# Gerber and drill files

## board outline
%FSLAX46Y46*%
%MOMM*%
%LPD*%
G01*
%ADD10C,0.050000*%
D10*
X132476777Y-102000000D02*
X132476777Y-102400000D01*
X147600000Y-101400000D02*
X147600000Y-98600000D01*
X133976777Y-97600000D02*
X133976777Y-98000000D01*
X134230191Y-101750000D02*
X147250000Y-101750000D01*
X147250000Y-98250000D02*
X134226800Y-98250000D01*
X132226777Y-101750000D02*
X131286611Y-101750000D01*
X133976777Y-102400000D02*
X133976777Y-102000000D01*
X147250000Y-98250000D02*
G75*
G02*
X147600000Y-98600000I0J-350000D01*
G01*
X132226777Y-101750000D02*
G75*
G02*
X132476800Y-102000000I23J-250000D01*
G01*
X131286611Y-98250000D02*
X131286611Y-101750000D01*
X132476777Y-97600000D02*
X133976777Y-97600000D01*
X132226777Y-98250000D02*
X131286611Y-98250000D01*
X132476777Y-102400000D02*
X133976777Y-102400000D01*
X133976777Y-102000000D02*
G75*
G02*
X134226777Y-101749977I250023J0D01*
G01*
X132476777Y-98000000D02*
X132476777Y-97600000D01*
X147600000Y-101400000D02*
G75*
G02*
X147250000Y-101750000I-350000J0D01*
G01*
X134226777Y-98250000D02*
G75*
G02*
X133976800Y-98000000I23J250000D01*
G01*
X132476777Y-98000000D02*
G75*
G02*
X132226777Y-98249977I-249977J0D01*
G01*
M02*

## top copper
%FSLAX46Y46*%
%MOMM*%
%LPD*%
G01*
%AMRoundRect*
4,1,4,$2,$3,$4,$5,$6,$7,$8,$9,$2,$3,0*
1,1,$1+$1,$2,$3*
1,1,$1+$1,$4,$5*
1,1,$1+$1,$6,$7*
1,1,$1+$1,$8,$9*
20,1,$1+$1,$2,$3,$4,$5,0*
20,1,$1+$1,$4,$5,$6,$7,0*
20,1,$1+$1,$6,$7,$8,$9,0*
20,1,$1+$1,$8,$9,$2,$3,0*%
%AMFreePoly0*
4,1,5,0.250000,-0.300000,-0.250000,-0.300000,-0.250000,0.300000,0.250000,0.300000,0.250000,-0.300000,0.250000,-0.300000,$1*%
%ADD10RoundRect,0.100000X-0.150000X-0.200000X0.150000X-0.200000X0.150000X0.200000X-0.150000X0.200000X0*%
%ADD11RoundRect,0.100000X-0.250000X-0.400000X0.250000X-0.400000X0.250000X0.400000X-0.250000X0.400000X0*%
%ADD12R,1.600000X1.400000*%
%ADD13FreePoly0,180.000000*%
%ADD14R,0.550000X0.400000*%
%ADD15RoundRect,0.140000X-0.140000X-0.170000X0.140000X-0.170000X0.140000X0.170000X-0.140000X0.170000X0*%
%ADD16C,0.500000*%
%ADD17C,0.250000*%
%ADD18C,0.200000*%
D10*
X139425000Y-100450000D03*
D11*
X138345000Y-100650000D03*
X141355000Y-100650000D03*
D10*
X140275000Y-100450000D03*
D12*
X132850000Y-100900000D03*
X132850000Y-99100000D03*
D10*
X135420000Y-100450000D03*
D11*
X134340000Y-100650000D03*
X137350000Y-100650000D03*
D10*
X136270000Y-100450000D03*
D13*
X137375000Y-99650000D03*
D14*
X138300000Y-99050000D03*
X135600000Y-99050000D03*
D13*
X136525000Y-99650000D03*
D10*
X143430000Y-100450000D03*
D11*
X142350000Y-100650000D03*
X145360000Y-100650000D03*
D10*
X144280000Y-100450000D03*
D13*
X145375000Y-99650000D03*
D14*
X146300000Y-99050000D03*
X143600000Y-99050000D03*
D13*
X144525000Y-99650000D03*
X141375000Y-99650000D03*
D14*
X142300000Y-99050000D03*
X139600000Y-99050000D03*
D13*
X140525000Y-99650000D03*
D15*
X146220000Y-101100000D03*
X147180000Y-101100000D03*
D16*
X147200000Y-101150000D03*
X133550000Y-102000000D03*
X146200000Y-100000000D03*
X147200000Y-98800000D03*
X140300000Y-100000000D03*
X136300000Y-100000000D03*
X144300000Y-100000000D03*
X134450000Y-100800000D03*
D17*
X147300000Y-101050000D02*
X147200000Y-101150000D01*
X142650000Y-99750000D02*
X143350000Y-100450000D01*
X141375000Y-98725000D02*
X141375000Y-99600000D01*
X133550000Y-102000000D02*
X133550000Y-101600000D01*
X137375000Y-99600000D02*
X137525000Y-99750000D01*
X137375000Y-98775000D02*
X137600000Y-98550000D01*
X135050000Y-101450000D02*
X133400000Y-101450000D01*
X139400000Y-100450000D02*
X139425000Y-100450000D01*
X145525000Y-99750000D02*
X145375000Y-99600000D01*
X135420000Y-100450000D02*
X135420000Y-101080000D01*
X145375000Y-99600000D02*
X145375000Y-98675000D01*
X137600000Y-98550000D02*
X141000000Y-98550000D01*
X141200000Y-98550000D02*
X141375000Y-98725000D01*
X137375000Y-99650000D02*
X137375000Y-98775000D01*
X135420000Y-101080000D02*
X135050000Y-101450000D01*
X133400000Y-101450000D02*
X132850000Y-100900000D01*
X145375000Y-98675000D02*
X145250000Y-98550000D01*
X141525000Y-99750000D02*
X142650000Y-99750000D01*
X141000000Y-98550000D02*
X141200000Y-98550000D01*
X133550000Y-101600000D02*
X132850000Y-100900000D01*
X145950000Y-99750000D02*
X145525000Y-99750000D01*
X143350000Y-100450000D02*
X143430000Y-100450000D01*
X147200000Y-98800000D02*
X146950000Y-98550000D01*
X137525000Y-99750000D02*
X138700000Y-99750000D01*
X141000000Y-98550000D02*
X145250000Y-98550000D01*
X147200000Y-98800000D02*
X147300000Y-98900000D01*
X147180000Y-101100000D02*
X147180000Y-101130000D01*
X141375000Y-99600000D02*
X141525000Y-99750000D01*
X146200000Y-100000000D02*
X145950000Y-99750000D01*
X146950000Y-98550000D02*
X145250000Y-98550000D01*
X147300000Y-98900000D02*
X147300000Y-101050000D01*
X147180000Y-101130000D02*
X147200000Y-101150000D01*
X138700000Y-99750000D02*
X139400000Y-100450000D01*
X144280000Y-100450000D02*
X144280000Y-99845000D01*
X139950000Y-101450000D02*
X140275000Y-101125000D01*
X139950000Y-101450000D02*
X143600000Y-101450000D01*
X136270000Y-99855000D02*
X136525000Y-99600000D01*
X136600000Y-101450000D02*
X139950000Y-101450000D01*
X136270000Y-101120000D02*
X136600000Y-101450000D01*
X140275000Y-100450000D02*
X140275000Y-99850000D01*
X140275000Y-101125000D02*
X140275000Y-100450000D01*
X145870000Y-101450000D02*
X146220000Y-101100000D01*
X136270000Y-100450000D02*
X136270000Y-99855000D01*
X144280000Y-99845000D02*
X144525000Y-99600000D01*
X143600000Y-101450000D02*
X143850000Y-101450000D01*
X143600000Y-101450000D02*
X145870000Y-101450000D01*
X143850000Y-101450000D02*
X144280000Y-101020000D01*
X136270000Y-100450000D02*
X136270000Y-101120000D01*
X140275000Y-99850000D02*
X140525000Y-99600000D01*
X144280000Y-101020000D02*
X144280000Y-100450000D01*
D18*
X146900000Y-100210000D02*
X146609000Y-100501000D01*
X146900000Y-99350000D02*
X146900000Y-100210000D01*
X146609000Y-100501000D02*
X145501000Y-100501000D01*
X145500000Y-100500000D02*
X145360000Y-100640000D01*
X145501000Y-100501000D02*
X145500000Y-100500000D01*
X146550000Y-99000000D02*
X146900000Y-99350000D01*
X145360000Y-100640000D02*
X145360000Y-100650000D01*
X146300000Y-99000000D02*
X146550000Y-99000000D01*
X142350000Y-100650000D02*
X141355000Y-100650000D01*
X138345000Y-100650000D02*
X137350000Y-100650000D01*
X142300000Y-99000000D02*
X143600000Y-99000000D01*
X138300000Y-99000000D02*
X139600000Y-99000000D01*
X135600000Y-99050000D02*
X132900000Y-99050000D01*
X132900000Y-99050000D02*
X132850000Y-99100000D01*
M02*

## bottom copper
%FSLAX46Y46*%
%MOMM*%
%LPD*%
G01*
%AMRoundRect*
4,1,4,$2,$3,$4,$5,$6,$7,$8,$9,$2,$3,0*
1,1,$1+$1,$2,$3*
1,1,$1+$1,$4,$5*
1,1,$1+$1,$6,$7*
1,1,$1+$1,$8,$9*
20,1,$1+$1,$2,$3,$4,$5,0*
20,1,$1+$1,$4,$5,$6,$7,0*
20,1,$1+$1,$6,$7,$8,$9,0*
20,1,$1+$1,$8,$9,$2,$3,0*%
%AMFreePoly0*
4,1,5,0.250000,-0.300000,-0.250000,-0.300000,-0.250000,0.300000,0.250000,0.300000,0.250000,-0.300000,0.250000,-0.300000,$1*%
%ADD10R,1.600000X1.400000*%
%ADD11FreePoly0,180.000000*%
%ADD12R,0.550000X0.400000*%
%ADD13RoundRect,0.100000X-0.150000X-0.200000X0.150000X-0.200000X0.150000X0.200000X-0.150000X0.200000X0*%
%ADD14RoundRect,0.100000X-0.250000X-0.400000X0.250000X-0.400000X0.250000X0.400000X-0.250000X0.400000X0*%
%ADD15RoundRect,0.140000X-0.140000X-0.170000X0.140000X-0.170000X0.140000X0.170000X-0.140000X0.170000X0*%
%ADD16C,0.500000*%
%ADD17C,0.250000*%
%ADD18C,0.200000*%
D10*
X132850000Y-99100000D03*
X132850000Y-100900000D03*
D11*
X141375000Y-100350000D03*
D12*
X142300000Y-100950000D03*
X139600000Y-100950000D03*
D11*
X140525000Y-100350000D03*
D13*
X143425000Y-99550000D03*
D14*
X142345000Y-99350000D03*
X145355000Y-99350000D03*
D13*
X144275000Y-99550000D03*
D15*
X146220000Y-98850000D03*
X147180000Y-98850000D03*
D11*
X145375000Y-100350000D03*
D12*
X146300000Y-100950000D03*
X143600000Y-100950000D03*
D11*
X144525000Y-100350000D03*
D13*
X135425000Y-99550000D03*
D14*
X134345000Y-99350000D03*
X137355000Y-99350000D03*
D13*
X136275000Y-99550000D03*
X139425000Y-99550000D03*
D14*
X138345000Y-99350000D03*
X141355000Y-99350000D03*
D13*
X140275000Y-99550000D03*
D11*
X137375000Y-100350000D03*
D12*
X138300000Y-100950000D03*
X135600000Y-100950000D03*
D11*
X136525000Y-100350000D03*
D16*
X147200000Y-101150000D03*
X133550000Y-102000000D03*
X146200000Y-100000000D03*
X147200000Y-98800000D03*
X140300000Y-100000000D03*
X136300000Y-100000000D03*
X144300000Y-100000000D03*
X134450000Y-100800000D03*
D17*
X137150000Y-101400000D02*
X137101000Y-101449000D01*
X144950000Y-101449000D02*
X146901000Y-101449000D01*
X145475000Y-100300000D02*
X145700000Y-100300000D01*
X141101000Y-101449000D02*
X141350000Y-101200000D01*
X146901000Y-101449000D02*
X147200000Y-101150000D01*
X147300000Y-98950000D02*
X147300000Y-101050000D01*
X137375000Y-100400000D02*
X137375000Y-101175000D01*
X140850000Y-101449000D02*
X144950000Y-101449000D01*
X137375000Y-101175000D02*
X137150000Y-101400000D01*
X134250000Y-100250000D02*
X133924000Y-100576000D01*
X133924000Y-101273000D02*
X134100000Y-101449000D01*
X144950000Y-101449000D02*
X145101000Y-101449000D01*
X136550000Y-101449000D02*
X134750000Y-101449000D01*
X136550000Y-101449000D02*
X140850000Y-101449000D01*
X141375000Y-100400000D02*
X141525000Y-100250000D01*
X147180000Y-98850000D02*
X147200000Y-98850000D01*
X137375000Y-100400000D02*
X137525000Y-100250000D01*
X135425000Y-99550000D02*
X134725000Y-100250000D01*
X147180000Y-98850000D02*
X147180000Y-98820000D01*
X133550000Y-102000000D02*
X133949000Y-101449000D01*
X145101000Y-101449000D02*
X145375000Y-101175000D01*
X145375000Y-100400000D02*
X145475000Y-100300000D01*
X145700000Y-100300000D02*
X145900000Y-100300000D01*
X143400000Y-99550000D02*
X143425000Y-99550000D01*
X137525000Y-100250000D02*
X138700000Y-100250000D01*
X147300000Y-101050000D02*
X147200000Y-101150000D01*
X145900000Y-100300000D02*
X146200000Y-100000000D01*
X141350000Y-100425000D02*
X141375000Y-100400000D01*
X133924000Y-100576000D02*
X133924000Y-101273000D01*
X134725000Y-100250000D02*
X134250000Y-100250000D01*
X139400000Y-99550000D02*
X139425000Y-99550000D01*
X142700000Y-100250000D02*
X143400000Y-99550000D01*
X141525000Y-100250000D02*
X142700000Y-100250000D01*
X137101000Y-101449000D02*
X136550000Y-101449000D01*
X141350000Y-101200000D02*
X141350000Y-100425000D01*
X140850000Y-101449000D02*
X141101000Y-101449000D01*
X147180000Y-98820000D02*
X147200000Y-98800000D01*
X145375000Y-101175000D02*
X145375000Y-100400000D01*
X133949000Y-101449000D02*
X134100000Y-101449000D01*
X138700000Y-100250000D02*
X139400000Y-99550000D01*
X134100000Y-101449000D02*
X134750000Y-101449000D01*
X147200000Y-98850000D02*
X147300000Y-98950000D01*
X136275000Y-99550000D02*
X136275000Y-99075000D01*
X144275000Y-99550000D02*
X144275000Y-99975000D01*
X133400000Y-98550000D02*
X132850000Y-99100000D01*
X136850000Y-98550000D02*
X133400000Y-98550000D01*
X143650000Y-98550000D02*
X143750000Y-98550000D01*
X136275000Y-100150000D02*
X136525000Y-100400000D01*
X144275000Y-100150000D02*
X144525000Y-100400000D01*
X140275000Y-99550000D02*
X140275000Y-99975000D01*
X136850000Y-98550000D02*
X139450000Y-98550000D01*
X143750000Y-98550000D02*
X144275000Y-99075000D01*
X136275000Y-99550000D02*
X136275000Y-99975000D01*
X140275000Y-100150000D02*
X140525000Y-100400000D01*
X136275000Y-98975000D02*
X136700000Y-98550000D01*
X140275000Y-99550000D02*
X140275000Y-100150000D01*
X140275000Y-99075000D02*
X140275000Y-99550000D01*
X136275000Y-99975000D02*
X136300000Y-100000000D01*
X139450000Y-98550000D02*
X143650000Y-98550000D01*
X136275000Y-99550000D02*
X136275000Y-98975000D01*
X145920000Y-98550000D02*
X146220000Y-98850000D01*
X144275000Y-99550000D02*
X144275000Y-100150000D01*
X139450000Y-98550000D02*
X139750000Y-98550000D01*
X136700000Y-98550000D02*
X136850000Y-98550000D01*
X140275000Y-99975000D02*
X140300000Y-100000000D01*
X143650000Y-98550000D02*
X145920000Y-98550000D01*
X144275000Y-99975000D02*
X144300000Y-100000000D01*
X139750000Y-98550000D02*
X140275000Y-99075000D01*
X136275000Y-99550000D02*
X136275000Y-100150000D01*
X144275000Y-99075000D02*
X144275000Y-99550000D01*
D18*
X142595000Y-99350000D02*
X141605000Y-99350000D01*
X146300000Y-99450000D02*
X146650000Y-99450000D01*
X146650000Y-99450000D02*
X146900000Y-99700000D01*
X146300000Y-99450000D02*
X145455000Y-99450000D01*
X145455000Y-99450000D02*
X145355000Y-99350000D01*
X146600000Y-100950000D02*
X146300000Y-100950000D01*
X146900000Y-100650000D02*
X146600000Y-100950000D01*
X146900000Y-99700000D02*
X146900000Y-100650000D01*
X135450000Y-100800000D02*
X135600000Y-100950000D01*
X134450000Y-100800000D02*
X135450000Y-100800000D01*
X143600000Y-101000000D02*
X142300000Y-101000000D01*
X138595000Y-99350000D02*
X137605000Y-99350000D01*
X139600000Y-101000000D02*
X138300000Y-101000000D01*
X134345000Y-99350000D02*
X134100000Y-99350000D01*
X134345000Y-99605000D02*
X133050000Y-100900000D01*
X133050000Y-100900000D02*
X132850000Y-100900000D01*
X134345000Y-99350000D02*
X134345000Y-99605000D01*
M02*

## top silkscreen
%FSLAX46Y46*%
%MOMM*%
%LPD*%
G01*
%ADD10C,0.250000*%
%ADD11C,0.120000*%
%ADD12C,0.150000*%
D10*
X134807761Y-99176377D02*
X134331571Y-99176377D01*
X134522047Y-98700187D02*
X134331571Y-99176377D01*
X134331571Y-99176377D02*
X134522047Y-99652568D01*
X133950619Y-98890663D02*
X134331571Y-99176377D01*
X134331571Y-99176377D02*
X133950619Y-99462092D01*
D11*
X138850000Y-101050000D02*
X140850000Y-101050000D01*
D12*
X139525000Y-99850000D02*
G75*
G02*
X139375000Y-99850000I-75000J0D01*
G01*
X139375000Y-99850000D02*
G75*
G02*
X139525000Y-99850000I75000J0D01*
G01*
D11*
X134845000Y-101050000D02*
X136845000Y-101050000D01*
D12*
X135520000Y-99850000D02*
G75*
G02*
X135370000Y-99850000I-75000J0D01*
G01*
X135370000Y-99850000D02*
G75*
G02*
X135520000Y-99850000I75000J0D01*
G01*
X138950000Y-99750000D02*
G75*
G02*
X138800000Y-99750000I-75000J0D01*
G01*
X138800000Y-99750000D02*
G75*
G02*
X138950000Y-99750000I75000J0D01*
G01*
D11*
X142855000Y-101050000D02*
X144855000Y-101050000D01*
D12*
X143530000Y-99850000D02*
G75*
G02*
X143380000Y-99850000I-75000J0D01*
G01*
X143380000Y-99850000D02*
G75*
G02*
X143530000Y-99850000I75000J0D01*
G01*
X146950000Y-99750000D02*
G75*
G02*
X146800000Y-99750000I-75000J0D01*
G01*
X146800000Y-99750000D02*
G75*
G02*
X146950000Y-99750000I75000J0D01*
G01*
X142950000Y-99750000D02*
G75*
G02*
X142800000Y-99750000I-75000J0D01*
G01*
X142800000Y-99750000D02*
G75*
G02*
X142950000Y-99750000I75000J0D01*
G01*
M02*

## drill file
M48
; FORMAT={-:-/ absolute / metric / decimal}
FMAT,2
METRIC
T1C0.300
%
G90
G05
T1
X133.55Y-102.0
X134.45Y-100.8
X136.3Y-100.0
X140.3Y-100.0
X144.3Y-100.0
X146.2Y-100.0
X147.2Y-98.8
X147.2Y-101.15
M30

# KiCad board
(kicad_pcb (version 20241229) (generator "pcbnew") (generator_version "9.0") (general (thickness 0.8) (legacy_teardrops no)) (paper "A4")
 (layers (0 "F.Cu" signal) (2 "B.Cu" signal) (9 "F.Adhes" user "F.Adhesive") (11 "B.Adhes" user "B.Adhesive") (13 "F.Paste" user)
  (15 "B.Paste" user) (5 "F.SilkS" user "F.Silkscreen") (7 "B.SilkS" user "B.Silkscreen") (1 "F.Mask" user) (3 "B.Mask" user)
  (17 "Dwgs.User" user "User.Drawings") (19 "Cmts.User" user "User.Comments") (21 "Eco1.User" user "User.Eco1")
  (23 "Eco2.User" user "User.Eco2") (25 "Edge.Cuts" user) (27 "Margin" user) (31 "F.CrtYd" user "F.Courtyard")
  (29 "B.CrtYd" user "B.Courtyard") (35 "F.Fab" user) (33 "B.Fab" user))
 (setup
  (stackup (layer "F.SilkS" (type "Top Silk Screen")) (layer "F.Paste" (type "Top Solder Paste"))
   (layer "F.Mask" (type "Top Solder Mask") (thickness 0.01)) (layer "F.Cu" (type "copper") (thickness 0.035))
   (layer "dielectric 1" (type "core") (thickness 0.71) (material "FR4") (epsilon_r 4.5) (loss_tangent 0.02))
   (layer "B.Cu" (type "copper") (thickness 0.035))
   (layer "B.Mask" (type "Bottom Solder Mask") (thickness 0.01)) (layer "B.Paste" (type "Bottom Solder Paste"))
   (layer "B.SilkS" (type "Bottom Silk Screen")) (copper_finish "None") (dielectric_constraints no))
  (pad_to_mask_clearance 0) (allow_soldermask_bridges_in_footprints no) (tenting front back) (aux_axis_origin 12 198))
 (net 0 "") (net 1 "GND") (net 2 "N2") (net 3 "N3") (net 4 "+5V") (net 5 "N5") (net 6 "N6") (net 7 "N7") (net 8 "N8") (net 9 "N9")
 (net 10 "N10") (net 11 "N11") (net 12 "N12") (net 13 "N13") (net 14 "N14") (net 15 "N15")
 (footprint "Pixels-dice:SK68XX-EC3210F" (layer "F.Cu") (at 139.85 100.65)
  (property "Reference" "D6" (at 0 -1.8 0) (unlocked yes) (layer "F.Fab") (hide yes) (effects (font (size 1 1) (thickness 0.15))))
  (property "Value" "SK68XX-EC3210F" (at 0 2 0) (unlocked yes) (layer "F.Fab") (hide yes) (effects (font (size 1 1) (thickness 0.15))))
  (fp_line (start -1 0.4) (end 1 0.4) (stroke (width 0.12) (type default)) (layer "F.SilkS"))
  (fp_circle (center -0.4 -0.8) (end -0.3 -0.8) (stroke (width 0.1) (type solid)) (fill yes) (layer "F.SilkS"))
  (pad "1" smd roundrect (at -0.425 -0.2) (size 0.5 0.6) (layers "F.Cu" "F.Mask" "F.Paste") (roundrect_rratio 0.2) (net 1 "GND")
   (thermal_bridge_angle 45))
  (pad "2" smd roundrect (at -1.505 0) (size 0.7 1) (layers "F.Cu" "F.Mask" "F.Paste") (roundrect_rratio 0.1428571429) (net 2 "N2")
   (thermal_bridge_angle 45))
  (pad "3" smd roundrect (at 1.505 0) (size 0.7 1) (layers "F.Cu" "F.Mask" "F.Paste") (roundrect_rratio 0.1428571429) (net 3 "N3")
   (thermal_bridge_angle 45))
  (pad "4" smd roundrect (at 0.425 -0.2) (size 0.5 0.6) (layers "F.Cu" "F.Mask" "F.Paste") (roundrect_rratio 0.2) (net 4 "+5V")
   (thermal_bridge_angle 45)))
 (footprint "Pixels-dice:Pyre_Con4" (layer "F.Cu") (at 132.85 100 90)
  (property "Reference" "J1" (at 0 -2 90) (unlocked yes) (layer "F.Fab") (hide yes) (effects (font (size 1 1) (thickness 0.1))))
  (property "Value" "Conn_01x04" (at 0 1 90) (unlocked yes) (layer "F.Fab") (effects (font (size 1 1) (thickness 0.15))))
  (pad "1" connect rect (at -0.9 0 90) (size 1.4 1.6) (layers "F.Cu" "F.Mask") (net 1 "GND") (thermal_bridge_angle 45))
  (pad "2" connect rect (at 0.9 0 90) (size 1.4 1.6) (layers "F.Cu" "F.Mask") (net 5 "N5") (thermal_bridge_angle 45))
  (pad "3" connect rect (at 0.9 0 90) (size 1.4 1.6) (layers "B.Cu" "B.Mask") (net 4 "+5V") (thermal_bridge_angle 45))
  (pad "4" connect rect (at -0.9 0 90) (size 1.4 1.6) (layers "B.Cu" "B.Mask") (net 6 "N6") (thermal_bridge_angle 45)))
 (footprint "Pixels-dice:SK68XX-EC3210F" (layer "F.Cu") (at 135.845 100.65)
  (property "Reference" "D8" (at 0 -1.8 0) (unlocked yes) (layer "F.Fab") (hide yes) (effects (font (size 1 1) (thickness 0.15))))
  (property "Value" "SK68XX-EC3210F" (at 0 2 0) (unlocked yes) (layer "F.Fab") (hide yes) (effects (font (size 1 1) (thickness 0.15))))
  (fp_line (start -1 0.4) (end 1 0.4) (stroke (width 0.12) (type default)) (layer "F.SilkS"))
  (fp_circle (center -0.4 -0.8) (end -0.3 -0.8) (stroke (width 0.1) (type solid)) (fill yes) (layer "F.SilkS"))
  (pad "1" smd roundrect (at -0.425 -0.2) (size 0.5 0.6) (layers "F.Cu" "F.Mask" "F.Paste") (roundrect_rratio 0.2) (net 1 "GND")
   (thermal_bridge_angle 45))
  (pad "2" smd roundrect (at -1.505 0) (size 0.7 1) (layers "F.Cu" "F.Mask" "F.Paste") (roundrect_rratio 0.1428571429) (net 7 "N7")
   (thermal_bridge_angle 45))
  (pad "3" smd roundrect (at 1.505 0) (size 0.7 1) (layers "F.Cu" "F.Mask" "F.Paste") (roundrect_rratio 0.1428571429) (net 2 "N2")
   (thermal_bridge_angle 45))
  (pad "4" smd roundrect (at 0.425 -0.2) (size 0.5 0.6) (layers "F.Cu" "F.Mask" "F.Paste") (roundrect_rratio 0.2) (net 4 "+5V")
   (thermal_bridge_angle 45)))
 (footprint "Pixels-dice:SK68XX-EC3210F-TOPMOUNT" (layer "F.Cu") (at 136.95 99.4 180)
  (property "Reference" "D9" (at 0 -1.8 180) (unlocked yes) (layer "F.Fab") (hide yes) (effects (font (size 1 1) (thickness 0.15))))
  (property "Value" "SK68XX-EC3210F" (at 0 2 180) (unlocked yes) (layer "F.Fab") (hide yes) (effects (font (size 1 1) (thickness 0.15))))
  (fp_circle (center -1.925 -0.35) (end -1.825 -0.35) (stroke (width 0.1) (type solid)) (fill yes) (layer "F.SilkS"))
  (pad "1" smd custom (at -0.425 -0.25 180) (size 0.5 0.6) (layers "F.Cu" "F.Mask" "F.Paste") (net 1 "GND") (thermal_bridge_angle 45)
   (options (clearance outline) (anchor rect)) (primitives))
  (pad "2" smd rect (at -1.35 0.35 180) (size 0.55 0.4) (layers "F.Cu" "F.Mask" "F.Paste") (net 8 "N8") (thermal_bridge_angle 45))
  (pad "3" smd rect (at 1.35 0.35 180) (size 0.55 0.4) (layers "F.Cu" "F.Mask" "F.Paste") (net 5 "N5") (thermal_bridge_angle 45))
  (pad "4" smd custom (at 0.425 -0.25 180) (size 0.5 0.6) (layers "F.Cu" "F.Mask" "F.Paste") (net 4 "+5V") (thermal_bridge_angle 45)
   (options (clearance outline) (anchor rect)) (primitives)))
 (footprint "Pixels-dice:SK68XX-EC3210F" (layer "F.Cu") (at 143.855 100.65)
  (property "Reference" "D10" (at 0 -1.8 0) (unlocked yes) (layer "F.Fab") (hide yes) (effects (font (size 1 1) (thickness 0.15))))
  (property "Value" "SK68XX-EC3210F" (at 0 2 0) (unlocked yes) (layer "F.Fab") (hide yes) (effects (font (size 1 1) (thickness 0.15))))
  (fp_line (start -1 0.4) (end 1 0.4) (stroke (width 0.12) (type default)) (layer "F.SilkS"))
  (fp_circle (center -0.4 -0.8) (end -0.3 -0.8) (stroke (width 0.1) (type solid)) (fill yes) (layer "F.SilkS"))
  (pad "1" smd roundrect (at -0.425 -0.2) (size 0.5 0.6) (layers "F.Cu" "F.Mask" "F.Paste") (roundrect_rratio 0.2) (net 1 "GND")
   (thermal_bridge_angle 45))
  (pad "2" smd roundrect (at -1.505 0) (size 0.7 1) (layers "F.Cu" "F.Mask" "F.Paste") (roundrect_rratio 0.1428571429) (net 3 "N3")
   (thermal_bridge_angle 45))
  (pad "3" smd roundrect (at 1.505 0) (size 0.7 1) (layers "F.Cu" "F.Mask" "F.Paste") (roundrect_rratio 0.1428571429) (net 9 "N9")
   (thermal_bridge_angle 45))
  (pad "4" smd roundrect (at 0.425 -0.2) (size 0.5 0.6) (layers "F.Cu" "F.Mask" "F.Paste") (roundrect_rratio 0.2) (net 4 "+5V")
   (thermal_bridge_angle 45)))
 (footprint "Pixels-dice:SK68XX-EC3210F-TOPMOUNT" (layer "F.Cu") (at 144.95 99.4 180)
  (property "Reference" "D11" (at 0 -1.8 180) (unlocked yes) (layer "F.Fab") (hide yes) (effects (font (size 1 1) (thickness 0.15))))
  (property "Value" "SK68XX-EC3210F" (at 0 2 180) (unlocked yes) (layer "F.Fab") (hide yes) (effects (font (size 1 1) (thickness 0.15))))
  (fp_circle (center -1.925 -0.35) (end -1.825 -0.35) (stroke (width 0.1) (type solid)) (fill yes) (layer "F.SilkS"))
  (pad "1" smd custom (at -0.425 -0.25 180) (size 0.5 0.6) (layers "F.Cu" "F.Mask" "F.Paste") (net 1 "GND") (thermal_bridge_angle 45)
   (options (clearance outline) (anchor rect)) (primitives))
  (pad "2" smd rect (at -1.35 0.35 180) (size 0.55 0.4) (layers "F.Cu" "F.Mask" "F.Paste") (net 9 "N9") (thermal_bridge_angle 45))
  (pad "3" smd rect (at 1.35 0.35 180) (size 0.55 0.4) (layers "F.Cu" "F.Mask" "F.Paste") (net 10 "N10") (thermal_bridge_angle 45))
  (pad "4" smd custom (at 0.425 -0.25 180) (size 0.5 0.6) (layers "F.Cu" "F.Mask" "F.Paste") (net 4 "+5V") (thermal_bridge_angle 45)
   (options (clearance outline) (anchor rect)) (primitives)))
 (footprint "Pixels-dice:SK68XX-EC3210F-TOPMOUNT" (layer "F.Cu") (at 140.95 99.4 180)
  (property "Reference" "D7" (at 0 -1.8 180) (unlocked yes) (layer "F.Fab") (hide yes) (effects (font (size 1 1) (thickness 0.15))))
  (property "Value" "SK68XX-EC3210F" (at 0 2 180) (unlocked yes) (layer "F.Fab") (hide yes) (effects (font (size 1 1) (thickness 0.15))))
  (fp_circle (center -1.925 -0.35) (end -1.825 -0.35) (stroke (width 0.1) (type solid)) (fill yes) (layer "F.SilkS"))
  (pad "1" smd custom (at -0.425 -0.25 180) (size 0.5 0.6) (layers "F.Cu" "F.Mask" "F.Paste") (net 1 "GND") (thermal_bridge_angle 45)
   (options (clearance outline) (anchor rect)) (primitives))
  (pad "2" smd rect (at -1.35 0.35 180) (size 0.55 0.4) (layers "F.Cu" "F.Mask" "F.Paste") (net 10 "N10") (thermal_bridge_angle 45))
  (pad "3" smd rect (at 1.35 0.35 180) (size 0.55 0.4) (layers "F.Cu" "F.Mask" "F.Paste") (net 8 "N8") (thermal_bridge_angle 45))
  (pad "4" smd custom (at 0.425 -0.25 180) (size 0.5 0.6) (layers "F.Cu" "F.Mask" "F.Paste") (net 4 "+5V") (thermal_bridge_angle 45)
   (options (clearance outline) (anchor rect)) (primitives)))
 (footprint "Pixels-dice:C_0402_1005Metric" (layer "F.Cu") (at 146.7 101.1)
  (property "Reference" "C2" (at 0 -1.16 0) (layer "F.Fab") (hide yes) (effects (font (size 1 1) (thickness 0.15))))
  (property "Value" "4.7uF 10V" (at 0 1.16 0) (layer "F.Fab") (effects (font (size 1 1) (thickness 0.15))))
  (pad "1" smd roundrect (at -0.48 0) (size 0.56 0.62) (layers "F.Cu" "F.Mask" "F.Paste") (roundrect_rratio 0.25) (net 4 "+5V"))
  (pad "2" smd roundrect (at 0.48 0) (size 0.56 0.62) (layers "F.Cu" "F.Mask" "F.Paste") (roundrect_rratio 0.25) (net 1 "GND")))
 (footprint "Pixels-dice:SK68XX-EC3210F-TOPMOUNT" (layer "B.Cu") (at 140.95 100.6 180)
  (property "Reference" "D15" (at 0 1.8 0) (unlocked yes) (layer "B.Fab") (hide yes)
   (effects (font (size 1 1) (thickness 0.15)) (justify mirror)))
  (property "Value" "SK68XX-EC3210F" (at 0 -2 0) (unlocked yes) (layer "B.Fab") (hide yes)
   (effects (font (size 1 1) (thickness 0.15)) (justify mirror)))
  (pad "1" smd custom (at -0.425 0.25 180) (size 0.5 0.6) (layers "B.Cu" "B.Mask" "B.Paste") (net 1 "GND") (thermal_bridge_angle 45)
   (options (clearance outline) (anchor rect)) (primitives))
  (pad "2" smd rect (at -1.35 -0.35 180) (size 0.55 0.4) (layers "B.Cu" "B.Mask" "B.Paste") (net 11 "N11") (thermal_bridge_angle 45))
  (pad "3" smd rect (at 1.35 -0.35 180) (size 0.55 0.4) (layers "B.Cu" "B.Mask" "B.Paste") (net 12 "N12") (thermal_bridge_angle 45))
  (pad "4" smd custom (at 0.425 0.25 180) (size 0.5 0.6) (layers "B.Cu" "B.Mask" "B.Paste") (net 4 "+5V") (thermal_bridge_angle 45)
   (options (clearance outline) (anchor rect)) (primitives)))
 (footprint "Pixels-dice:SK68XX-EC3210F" (layer "B.Cu") (at 143.85 99.35)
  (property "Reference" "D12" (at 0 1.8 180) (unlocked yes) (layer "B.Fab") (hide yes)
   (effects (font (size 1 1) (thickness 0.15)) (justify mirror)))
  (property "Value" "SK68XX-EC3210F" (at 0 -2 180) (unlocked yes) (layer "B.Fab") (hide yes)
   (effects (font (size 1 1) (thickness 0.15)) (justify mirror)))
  (pad "1" smd roundrect (at -0.425 0.2) (size 0.5 0.6) (layers "B.Cu" "B.Mask" "B.Paste") (roundrect_rratio 0.2) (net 1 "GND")
   (thermal_bridge_angle 45))
  (pad "2" smd roundrect (at -1.505 0) (size 0.7 1) (layers "B.Cu" "B.Mask" "B.Paste") (roundrect_rratio 0.1428571429) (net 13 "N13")
   (thermal_bridge_angle 45))
  (pad "3" smd roundrect (at 1.505 0) (size 0.7 1) (layers "B.Cu" "B.Mask" "B.Paste") (roundrect_rratio 0.1428571429) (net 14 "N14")
   (thermal_bridge_angle 45))
  (pad "4" smd roundrect (at 0.425 0.2) (size 0.5 0.6) (layers "B.Cu" "B.Mask" "B.Paste") (roundrect_rratio 0.2) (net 4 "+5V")
   (thermal_bridge_angle 45)))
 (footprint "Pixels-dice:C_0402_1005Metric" (layer "B.Cu") (at 146.7 98.85)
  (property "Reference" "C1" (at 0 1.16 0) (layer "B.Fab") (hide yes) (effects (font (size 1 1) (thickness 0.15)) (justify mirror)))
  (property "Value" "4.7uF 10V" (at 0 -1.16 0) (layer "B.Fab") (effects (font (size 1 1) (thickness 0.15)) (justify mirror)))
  (pad "1" smd roundrect (at -0.48 0) (size 0.56 0.62) (layers "B.Cu" "B.Mask" "B.Paste") (roundrect_rratio 0.25) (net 4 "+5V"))
  (pad "2" smd roundrect (at 0.48 0) (size 0.56 0.62) (layers "B.Cu" "B.Mask" "B.Paste") (roundrect_rratio 0.25) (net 1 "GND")))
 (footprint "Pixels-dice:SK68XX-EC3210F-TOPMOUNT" (layer "B.Cu") (at 144.95 100.6 180)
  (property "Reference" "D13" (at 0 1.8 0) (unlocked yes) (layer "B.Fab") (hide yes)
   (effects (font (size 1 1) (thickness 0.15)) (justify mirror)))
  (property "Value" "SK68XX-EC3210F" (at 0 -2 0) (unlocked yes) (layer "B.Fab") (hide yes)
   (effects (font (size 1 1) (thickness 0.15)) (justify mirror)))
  (pad "1" smd custom (at -0.425 0.25 180) (size 0.5 0.6) (layers "B.Cu" "B.Mask" "B.Paste") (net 1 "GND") (thermal_bridge_angle 45)
   (options (clearance outline) (anchor rect)) (primitives))
  (pad "2" smd rect (at -1.35 -0.35 180) (size 0.55 0.4) (layers "B.Cu" "B.Mask" "B.Paste") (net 14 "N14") (thermal_bridge_angle 45))
  (pad "3" smd rect (at 1.35 -0.35 180) (size 0.55 0.4) (layers "B.Cu" "B.Mask" "B.Paste") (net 11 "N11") (thermal_bridge_angle 45))
  (pad "4" smd custom (at 0.425 0.25 180) (size 0.5 0.6) (layers "B.Cu" "B.Mask" "B.Paste") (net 4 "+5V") (thermal_bridge_angle 45)
   (options (clearance outline) (anchor rect)) (primitives)))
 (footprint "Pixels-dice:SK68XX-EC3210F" (layer "B.Cu") (at 135.85 99.35)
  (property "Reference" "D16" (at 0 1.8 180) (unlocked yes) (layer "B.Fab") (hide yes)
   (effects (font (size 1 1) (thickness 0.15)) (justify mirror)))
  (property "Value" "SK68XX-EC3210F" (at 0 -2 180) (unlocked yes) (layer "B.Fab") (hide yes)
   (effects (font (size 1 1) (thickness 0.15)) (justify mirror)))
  (pad "1" smd roundrect (at -0.425 0.2) (size 0.5 0.6) (layers "B.Cu" "B.Mask" "B.Paste") (roundrect_rratio 0.2) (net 1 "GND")
   (thermal_bridge_angle 45))
  (pad "2" smd roundrect (at -1.505 0) (size 0.7 1) (layers "B.Cu" "B.Mask" "B.Paste") (roundrect_rratio 0.1428571429) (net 6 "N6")
   (thermal_bridge_angle 45))
  (pad "3" smd roundrect (at 1.505 0) (size 0.7 1) (layers "B.Cu" "B.Mask" "B.Paste") (roundrect_rratio 0.1428571429) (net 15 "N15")
   (thermal_bridge_angle 45))
  (pad "4" smd roundrect (at 0.425 0.2) (size 0.5 0.6) (layers "B.Cu" "B.Mask" "B.Paste") (roundrect_rratio 0.2) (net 4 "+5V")
   (thermal_bridge_angle 45)))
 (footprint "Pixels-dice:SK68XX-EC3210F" (layer "B.Cu") (at 139.85 99.35)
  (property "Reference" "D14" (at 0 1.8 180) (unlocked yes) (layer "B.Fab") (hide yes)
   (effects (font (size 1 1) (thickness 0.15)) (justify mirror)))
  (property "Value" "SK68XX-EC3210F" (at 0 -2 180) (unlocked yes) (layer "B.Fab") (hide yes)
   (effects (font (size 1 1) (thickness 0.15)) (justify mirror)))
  (pad "1" smd roundrect (at -0.425 0.2) (size 0.5 0.6) (layers "B.Cu" "B.Mask" "B.Paste") (roundrect_rratio 0.2) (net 1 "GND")
   (thermal_bridge_angle 45))
  (pad "2" smd roundrect (at -1.505 0) (size 0.7 1) (layers "B.Cu" "B.Mask" "B.Paste") (roundrect_rratio 0.1428571429) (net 15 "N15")
   (thermal_bridge_angle 45))
  (pad "3" smd roundrect (at 1.505 0) (size 0.7 1) (layers "B.Cu" "B.Mask" "B.Paste") (roundrect_rratio 0.1428571429) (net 13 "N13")
   (thermal_bridge_angle 45))
  (pad "4" smd roundrect (at 0.425 0.2) (size 0.5 0.6) (layers "B.Cu" "B.Mask" "B.Paste") (roundrect_rratio 0.2) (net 4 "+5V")
   (thermal_bridge_angle 45)))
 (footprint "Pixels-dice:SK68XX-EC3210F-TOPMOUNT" (layer "B.Cu") (at 136.95 100.6 180)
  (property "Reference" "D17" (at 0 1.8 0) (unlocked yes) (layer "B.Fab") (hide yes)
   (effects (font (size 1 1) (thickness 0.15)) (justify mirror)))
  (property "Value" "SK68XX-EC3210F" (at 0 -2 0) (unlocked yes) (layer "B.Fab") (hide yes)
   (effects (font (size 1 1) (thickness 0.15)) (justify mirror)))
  (pad "1" smd custom (at -0.425 0.25 180) (size 0.5 0.6) (layers "B.Cu" "B.Mask" "B.Paste") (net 1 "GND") (thermal_bridge_angle 45)
   (options (clearance outline) (anchor rect)) (primitives))
  (pad "2" smd rect (at -1.35 -0.35 180) (size 0.55 0.4) (layers "B.Cu" "B.Mask" "B.Paste") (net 12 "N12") (thermal_bridge_angle 45))
  (pad "3" smd rect (at 1.35 -0.35 180) (size 0.55 0.4) (layers "B.Cu" "B.Mask" "B.Paste") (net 7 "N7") (thermal_bridge_angle 45))
  (pad "4" smd custom (at 0.425 0.25 180) (size 0.5 0.6) (layers "B.Cu" "B.Mask" "B.Paste") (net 4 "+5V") (thermal_bridge_angle 45)
   (options (clearance outline) (anchor rect)) (primitives)))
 (gr_line (start 132.476777 102) (end 132.476777 102.4) (stroke (width 0.05) (type default)) (layer "Edge.Cuts"))
 (gr_line (start 147.6 101.4) (end 147.6 98.6) (stroke (width 0.05) (type default)) (layer "Edge.Cuts"))
 (gr_line (start 133.976777 97.6) (end 133.976777 98) (stroke (width 0.05) (type default)) (layer "Edge.Cuts"))
 (gr_line (start 134.230191 101.75) (end 147.25 101.75) (stroke (width 0.05) (type default)) (layer "Edge.Cuts"))
 (gr_line (start 147.25 98.25) (end 134.2268 98.25) (stroke (width 0.05) (type default)) (layer "Edge.Cuts"))
 (gr_line (start 132.226777 101.75) (end 131.286611 101.75) (stroke (width 0.05) (type default)) (layer "Edge.Cuts"))
 (gr_line (start 133.976777 102.4) (end 133.976777 102) (stroke (width 0.05) (type default)) (layer "Edge.Cuts"))
 (gr_arc (start 147.25 98.25) (mid 147.497487 98.352513) (end 147.6 98.6) (stroke (width 0.05) (type default)) (layer "Edge.Cuts"))
 (gr_arc (start 132.226777 101.75) (mid 132.403554 101.823223) (end 132.476777 102) (stroke (width 0.05) (type default)) (layer "Edge.Cuts"))
 (gr_line (start 131.286611 98.25) (end 131.286611 101.75) (stroke (width 0.05) (type default)) (layer "Edge.Cuts"))
 (gr_line (start 132.476777 97.6) (end 133.976777 97.6) (stroke (width 0.05) (type default)) (layer "Edge.Cuts"))
 (gr_line (start 132.226777 98.25) (end 131.286611 98.25) (stroke (width 0.05) (type default)) (layer "Edge.Cuts"))
 (gr_line (start 132.476777 102.4) (end 133.976777 102.4) (stroke (width 0.05) (type default)) (layer "Edge.Cuts"))
 (gr_arc (start 133.976777 102) (mid 134.05 101.823223) (end 134.226777 101.75) (stroke (width 0.05) (type default)) (layer "Edge.Cuts"))
 (gr_line (start 132.476777 98) (end 132.476777 97.6) (stroke (width 0.05) (type default)) (layer "Edge.Cuts"))
 (gr_arc (start 147.6 101.4) (mid 147.497487 101.647487) (end 147.25 101.75) (stroke (width 0.05) (type default)) (layer "Edge.Cuts"))
 (gr_arc (start 134.226777 98.25) (mid 134.05 98.176777) (end 133.976777 98) (stroke (width 0.05) (type default)) (layer "Edge.Cuts"))
 (gr_arc (start 132.476777 98) (mid 132.403554 98.176777) (end 132.226777 98.25) (stroke (width 0.05) (type default)) (layer "Edge.Cuts"))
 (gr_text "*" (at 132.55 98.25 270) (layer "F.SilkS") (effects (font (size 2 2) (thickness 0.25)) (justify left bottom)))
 (segment (start 147.3 101.05) (end 147.2 101.15) (width 0.25) (layer "F.Cu") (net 1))
 (segment (start 142.65 99.75) (end 143.35 100.45) (width 0.25) (layer "F.Cu") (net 1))
 (segment (start 141.375 98.725) (end 141.375 99.6) (width 0.25) (layer "F.Cu") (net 1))
 (segment (start 133.55 102) (end 133.55 101.6) (width 0.25) (layer "F.Cu") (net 1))
 (segment (start 137.375 99.6) (end 137.525 99.75) (width 0.25) (layer "F.Cu") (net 1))
 (segment (start 137.375 98.775) (end 137.6 98.55) (width 0.25) (layer "F.Cu") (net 1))
 (segment (start 135.05 101.45) (end 133.4 101.45) (width 0.25) (layer "F.Cu") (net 1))
 (segment (start 139.4 100.45) (end 139.425 100.45) (width 0.25) (layer "F.Cu") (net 1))
 (segment (start 145.525 99.75) (end 145.375 99.6) (width 0.25) (layer "F.Cu") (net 1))
 (segment (start 135.42 100.45) (end 135.42 101.08) (width 0.25) (layer "F.Cu") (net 1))
 (segment (start 145.375 99.6) (end 145.375 98.675) (width 0.25) (layer "F.Cu") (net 1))
 (segment (start 137.6 98.55) (end 141 98.55) (width 0.25) (layer "F.Cu") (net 1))
 (segment (start 141.2 98.55) (end 141.375 98.725) (width 0.25) (layer "F.Cu") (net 1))
 (segment (start 137.375 99.65) (end 137.375 98.775) (width 0.25) (layer "F.Cu") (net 1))
 (segment (start 135.42 101.08) (end 135.05 101.45) (width 0.25) (layer "F.Cu") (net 1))
 (segment (start 133.4 101.45) (end 132.85 100.9) (width 0.25) (layer "F.Cu") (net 1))
 (segment (start 145.375 98.675) (end 145.25 98.55) (width 0.25) (layer "F.Cu") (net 1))
 (segment (start 141.525 99.75) (end 142.65 99.75) (width 0.25) (layer "F.Cu") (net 1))
 (segment (start 141 98.55) (end 141.2 98.55) (width 0.25) (layer "F.Cu") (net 1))
 (segment (start 133.55 101.6) (end 132.85 100.9) (width 0.25) (layer "F.Cu") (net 1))
 (segment (start 145.95 99.75) (end 145.525 99.75) (width 0.25) (layer "F.Cu") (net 1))
 (segment (start 143.35 100.45) (end 143.43 100.45) (width 0.25) (layer "F.Cu") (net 1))
 (segment (start 147.2 98.8) (end 146.95 98.55) (width 0.25) (layer "F.Cu") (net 1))
 (segment (start 137.525 99.75) (end 138.7 99.75) (width 0.25) (layer "F.Cu") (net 1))
 (segment (start 141 98.55) (end 145.25 98.55) (width 0.25) (layer "F.Cu") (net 1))
 (segment (start 147.2 98.8) (end 147.3 98.9) (width 0.25) (layer "F.Cu") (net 1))
 (segment (start 147.18 101.1) (end 147.18 101.13) (width 0.25) (layer "F.Cu") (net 1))
 (segment (start 141.375 99.6) (end 141.525 99.75) (width 0.25) (layer "F.Cu") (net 1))
 (segment (start 146.2 100) (end 145.95 99.75) (width 0.25) (layer "F.Cu") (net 1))
 (segment (start 146.95 98.55) (end 145.25 98.55) (width 0.25) (layer "F.Cu") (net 1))
 (segment (start 147.3 98.9) (end 147.3 101.05) (width 0.25) (layer "F.Cu") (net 1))
 (segment (start 147.18 101.13) (end 147.2 101.15) (width 0.25) (layer "F.Cu") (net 1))
 (segment (start 138.7 99.75) (end 139.4 100.45) (width 0.25) (layer "F.Cu") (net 1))
 (via (at 147.2 101.15) (size 0.5) (drill 0.3) (layers "F.Cu" "B.Cu") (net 1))
 (via (at 133.55 102) (size 0.5) (drill 0.3) (layers "F.Cu" "B.Cu") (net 1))
 (via (at 146.2 100) (size 0.5) (drill 0.3) (layers "F.Cu" "B.Cu") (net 1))
 (via (at 147.2 98.8) (size 0.5) (drill 0.3) (layers "F.Cu" "B.Cu") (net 1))
 (segment (start 137.15 101.4) (end 137.101 101.449) (width 0.25) (layer "B.Cu") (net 1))
 (segment (start 144.95 101.449) (end 146.901 101.449) (width 0.25) (layer "B.Cu") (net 1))
 (segment (start 145.475 100.3) (end 145.7 100.3) (width 0.25) (layer "B.Cu") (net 1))
 (segment (start 141.101 101.449) (end 141.35 101.2) (width 0.25) (layer "B.Cu") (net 1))
 (segment (start 146.901 101.449) (end 147.2 101.15) (width 0.25) (layer "B.Cu") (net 1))
 (segment (start 147.3 98.95) (end 147.3 101.05) (width 0.25) (layer "B.Cu") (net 1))
 (segment (start 137.375 100.4) (end 137.375 101.175) (width 0.25) (layer "B.Cu") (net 1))
 (segment (start 140.85 101.449) (end 144.95 101.449) (width 0.25) (layer "B.Cu") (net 1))
 (segment (start 137.375 101.175) (end 137.15 101.4) (width 0.25) (layer "B.Cu") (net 1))
 (segment (start 134.25 100.25) (end 133.924 100.576) (width 0.25) (layer "B.Cu") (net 1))
 (segment (start 133.924 101.273) (end 134.1 101.449) (width 0.25) (layer "B.Cu") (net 1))
 (segment (start 144.95 101.449) (end 145.101 101.449) (width 0.25) (layer "B.Cu") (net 1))
 (segment (start 136.55 101.449) (end 134.75 101.449) (width 0.25) (layer "B.Cu") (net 1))
 (segment (start 136.55 101.449) (end 140.85 101.449) (width 0.25) (layer "B.Cu") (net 1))
 (segment (start 141.375 100.4) (end 141.525 100.25) (width 0.25) (layer "B.Cu") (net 1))
 (segment (start 147.18 98.85) (end 147.2 98.85) (width 0.25) (layer "B.Cu") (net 1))
 (segment (start 137.375 100.4) (end 137.525 100.25) (width 0.25) (layer "B.Cu") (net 1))
 (segment (start 135.425 99.55) (end 134.725 100.25) (width 0.25) (layer "B.Cu") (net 1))
 (segment (start 147.18 98.85) (end 147.18 98.82) (width 0.25) (layer "B.Cu") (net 1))
 (segment (start 133.55 102) (end 133.949 101.449) (width 0.25) (layer "B.Cu") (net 1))
 (segment (start 145.101 101.449) (end 145.375 101.175) (width 0.25) (layer "B.Cu") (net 1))
 (segment (start 145.375 100.4) (end 145.475 100.3) (width 0.25) (layer "B.Cu") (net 1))
 (segment (start 145.7 100.3) (end 145.9 100.3) (width 0.25) (layer "B.Cu") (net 1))
 (segment (start 143.4 99.55) (end 143.425 99.55) (width 0.25) (layer "B.Cu") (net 1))
 (segment (start 137.525 100.25) (end 138.7 100.25) (width 0.25) (layer "B.Cu") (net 1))
 (segment (start 147.3 101.05) (end 147.2 101.15) (width 0.25) (layer "B.Cu") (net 1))
 (segment (start 145.9 100.3) (end 146.2 100) (width 0.25) (layer "B.Cu") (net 1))
 (segment (start 141.35 100.425) (end 141.375 100.4) (width 0.25) (layer "B.Cu") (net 1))
 (segment (start 133.924 100.576) (end 133.924 101.273) (width 0.25) (layer "B.Cu") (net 1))
 (segment (start 134.725 100.25) (end 134.25 100.25) (width 0.25) (layer "B.Cu") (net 1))
 (segment (start 139.4 99.55) (end 139.425 99.55) (width 0.25) (layer "B.Cu") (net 1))
 (segment (start 142.7 100.25) (end 143.4 99.55) (width 0.25) (layer "B.Cu") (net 1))
 (segment (start 141.525 100.25) (end 142.7 100.25) (width 0.25) (layer "B.Cu") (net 1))
 (segment (start 137.101 101.449) (end 136.55 101.449) (width 0.25) (layer "B.Cu") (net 1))
 (segment (start 141.35 101.2) (end 141.35 100.425) (width 0.25) (layer "B.Cu") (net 1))
 (segment (start 140.85 101.449) (end 141.101 101.449) (width 0.25) (layer "B.Cu") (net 1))
 (segment (start 147.18 98.82) (end 147.2 98.8) (width 0.25) (layer "B.Cu") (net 1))
 (segment (start 145.375 101.175) (end 145.375 100.4) (width 0.25) (layer "B.Cu") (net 1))
 (segment (start 133.949 101.449) (end 134.1 101.449) (width 0.25) (layer "B.Cu") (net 1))
 (segment (start 138.7 100.25) (end 139.4 99.55) (width 0.25) (layer "B.Cu") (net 1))
 (segment (start 134.1 101.449) (end 134.75 101.449) (width 0.25) (layer "B.Cu") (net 1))
 (segment (start 147.2 98.85) (end 147.3 98.95) (width 0.25) (layer "B.Cu") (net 1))
 (segment (start 144.28 100.45) (end 144.28 99.845) (width 0.25) (layer "F.Cu") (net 4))
 (segment (start 139.95 101.45) (end 140.275 101.125) (width 0.25) (layer "F.Cu") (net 4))
 (segment (start 139.95 101.45) (end 143.6 101.45) (width 0.25) (layer "F.Cu") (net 4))
 (segment (start 136.27 99.855) (end 136.525 99.6) (width 0.25) (layer "F.Cu") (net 4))
 (segment (start 136.6 101.45) (end 139.95 101.45) (width 0.25) (layer "F.Cu") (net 4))
 (segment (start 136.27 101.12) (end 136.6 101.45) (width 0.25) (layer "F.Cu") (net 4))
 (segment (start 140.275 100.45) (end 140.275 99.85) (width 0.25) (layer "F.Cu") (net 4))
 (segment (start 140.275 101.125) (end 140.275 100.45) (width 0.25) (layer "F.Cu") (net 4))
 (segment (start 145.87 101.45) (end 146.22 101.1) (width 0.25) (layer "F.Cu") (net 4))
 (segment (start 136.27 100.45) (end 136.27 99.855) (width 0.25) (layer "F.Cu") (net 4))
 (segment (start 144.28 99.845) (end 144.525 99.6) (width 0.25) (layer "F.Cu") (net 4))
 (segment (start 143.6 101.45) (end 143.85 101.45) (width 0.25) (layer "F.Cu") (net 4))
 (segment (start 143.6 101.45) (end 145.87 101.45) (width 0.25) (layer "F.Cu") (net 4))
 (segment (start 143.85 101.45) (end 144.28 101.02) (width 0.25) (layer "F.Cu") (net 4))
 (segment (start 136.27 100.45) (end 136.27 101.12) (width 0.25) (layer "F.Cu") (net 4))
 (segment (start 140.275 99.85) (end 140.525 99.6) (width 0.25) (layer "F.Cu") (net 4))
 (segment (start 144.28 101.02) (end 144.28 100.45) (width 0.25) (layer "F.Cu") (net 4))
 (via (at 140.3 100) (size 0.5) (drill 0.3) (layers "F.Cu" "B.Cu") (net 4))
 (via (at 136.3 100) (size 0.5) (drill 0.3) (layers "F.Cu" "B.Cu") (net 4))
 (via (at 144.3 100) (size 0.5) (drill 0.3) (layers "F.Cu" "B.Cu") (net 4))
 (segment (start 136.275 99.55) (end 136.275 99.075) (width 0.25) (layer "B.Cu") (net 4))
 (segment (start 144.275 99.55) (end 144.275 99.975) (width 0.25) (layer "B.Cu") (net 4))
 (segment (start 133.4 98.55) (end 132.85 99.1) (width 0.25) (layer "B.Cu") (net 4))
 (segment (start 136.85 98.55) (end 133.4 98.55) (width 0.25) (layer "B.Cu") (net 4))
 (segment (start 143.65 98.55) (end 143.75 98.55) (width 0.25) (layer "B.Cu") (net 4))
 (segment (start 136.275 100.15) (end 136.525 100.4) (width 0.25) (layer "B.Cu") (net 4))
 (segment (start 144.275 100.15) (end 144.525 100.4) (width 0.25) (layer "B.Cu") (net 4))
 (segment (start 140.275 99.55) (end 140.275 99.975) (width 0.25) (layer "B.Cu") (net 4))
 (segment (start 136.85 98.55) (end 139.45 98.55) (width 0.25) (layer "B.Cu") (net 4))
 (segment (start 143.75 98.55) (end 144.275 99.075) (width 0.25) (layer "B.Cu") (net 4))
 (segment (start 136.275 99.55) (end 136.275 99.975) (width 0.25) (layer "B.Cu") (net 4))
 (segment (start 140.275 100.15) (end 140.525 100.4) (width 0.25) (layer "B.Cu") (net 4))
 (segment (start 136.275 98.975) (end 136.7 98.55) (width 0.25) (layer "B.Cu") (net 4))
 (segment (start 140.275 99.55) (end 140.275 100.15) (width 0.25) (layer "B.Cu") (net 4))
 (segment (start 140.275 99.075) (end 140.275 99.55) (width 0.25) (layer "B.Cu") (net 4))
 (segment (start 136.275 99.975) (end 136.3 100) (width 0.25) (layer "B.Cu") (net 4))
 (segment (start 139.45 98.55) (end 143.65 98.55) (width 0.25) (layer "B.Cu") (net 4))
 (segment (start 136.275 99.55) (end 136.275 98.975) (width 0.25) (layer "B.Cu") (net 4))
 (segment (start 145.92 98.55) (end 146.22 98.85) (width 0.25) (layer "B.Cu") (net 4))
 (segment (start 144.275 99.55) (end 144.275 100.15) (width 0.25) (layer "B.Cu") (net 4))
 (segment (start 139.45 98.55) (end 139.75 98.55) (width 0.25) (layer "B.Cu") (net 4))
 (segment (start 136.7 98.55) (end 136.85 98.55) (width 0.25) (layer "B.Cu") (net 4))
 (segment (start 140.275 99.975) (end 140.3 100) (width 0.25) (layer "B.Cu") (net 4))
 (segment (start 143.65 98.55) (end 145.92 98.55) (width 0.25) (layer "B.Cu") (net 4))
 (segment (start 144.275 99.975) (end 144.3 100) (width 0.25) (layer "B.Cu") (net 4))
 (segment (start 139.75 98.55) (end 140.275 99.075) (width 0.25) (layer "B.Cu") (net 4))
 (segment (start 136.275 99.55) (end 136.275 100.15) (width 0.25) (layer "B.Cu") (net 4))
 (segment (start 144.275 99.075) (end 144.275 99.55) (width 0.25) (layer "B.Cu") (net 4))
 (segment (start 146.9 100.21) (end 146.609 100.501) (width 0.2) (layer "F.Cu") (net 9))
 (segment (start 146.9 99.35) (end 146.9 100.21) (width 0.2) (layer "F.Cu") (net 9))
 (segment (start 146.609 100.501) (end 145.501 100.501) (width 0.2) (layer "F.Cu") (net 9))
 (segment (start 145.5 100.5) (end 145.36 100.64) (width 0.2) (layer "F.Cu") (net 9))
 (segment (start 145.501 100.501) (end 145.5 100.5) (width 0.2) (layer "F.Cu") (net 9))
 (segment (start 146.55 99) (end 146.9 99.35) (width 0.2) (layer "F.Cu") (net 9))
 (segment (start 145.36 100.64) (end 145.36 100.65) (width 0.2) (layer "F.Cu") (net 9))
 (segment (start 146.3 99) (end 146.55 99) (width 0.2) (layer "F.Cu") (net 9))
 (segment (start 142.35 100.65) (end 141.355 100.65) (width 0.2) (layer "F.Cu") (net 3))
 (segment (start 142.595 99.35) (end 141.605 99.35) (width 0.2) (layer "B.Cu") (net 13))
 (segment (start 146.3 99.45) (end 146.65 99.45) (width 0.2) (layer "B.Cu") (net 14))
 (segment (start 146.65 99.45) (end 146.9 99.7) (width 0.2) (layer "B.Cu") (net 14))
 (segment (start 146.3 99.45) (end 145.455 99.45) (width 0.2) (layer "B.Cu") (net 14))
 (segment (start 145.455 99.45) (end 145.355 99.35) (width 0.2) (layer "B.Cu") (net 14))
 (segment (start 146.6 100.95) (end 146.3 100.95) (width 0.2) (layer "B.Cu") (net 14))
 (segment (start 146.9 100.65) (end 146.6 100.95) (width 0.2) (layer "B.Cu") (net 14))
 (segment (start 146.9 99.7) (end 146.9 100.65) (width 0.2) (layer "B.Cu") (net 14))
 (segment (start 138.345 100.65) (end 137.35 100.65) (width 0.2) (layer "F.Cu") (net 2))
 (segment (start 142.3 99) (end 143.6 99) (width 0.2) (layer "F.Cu") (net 10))
 (segment (start 138.3 99) (end 139.6 99) (width 0.2) (layer "F.Cu") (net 8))
 (via (at 134.45 100.8) (size 0.5) (drill 0.3) (layers "F.Cu" "B.Cu") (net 7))
 (segment (start 135.45 100.8) (end 135.6 100.95) (width 0.2) (layer "B.Cu") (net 7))
 (segment (start 134.45 100.8) (end 135.45 100.8) (width 0.2) (layer "B.Cu") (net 7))
 (segment (start 143.6 101) (end 142.3 101) (width 0.2) (layer "B.Cu") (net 11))
 (segment (start 138.595 99.35) (end 137.605 99.35) (width 0.2) (layer "B.Cu") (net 15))
 (segment (start 139.6 101) (end 138.3 101) (width 0.2) (layer "B.Cu") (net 12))
 (segment (start 135.6 99.05) (end 132.9 99.05) (width 0.2) (layer "F.Cu") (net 5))
 (segment (start 132.9 99.05) (end 132.85 99.1) (width 0.2) (layer "F.Cu") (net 5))
 (segment (start 134.345 99.35) (end 134.1 99.35) (width 0.2) (layer "B.Cu") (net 6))
 (segment (start 134.345 99.605) (end 133.05 100.9) (width 0.2) (layer "B.Cu") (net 6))
 (segment (start 133.05 100.9) (end 132.85 100.9) (width 0.2) (layer "B.Cu") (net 6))
 (segment (start 134.345 99.35) (end 134.345 99.605) (width 0.2) (layer "B.Cu") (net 6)))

